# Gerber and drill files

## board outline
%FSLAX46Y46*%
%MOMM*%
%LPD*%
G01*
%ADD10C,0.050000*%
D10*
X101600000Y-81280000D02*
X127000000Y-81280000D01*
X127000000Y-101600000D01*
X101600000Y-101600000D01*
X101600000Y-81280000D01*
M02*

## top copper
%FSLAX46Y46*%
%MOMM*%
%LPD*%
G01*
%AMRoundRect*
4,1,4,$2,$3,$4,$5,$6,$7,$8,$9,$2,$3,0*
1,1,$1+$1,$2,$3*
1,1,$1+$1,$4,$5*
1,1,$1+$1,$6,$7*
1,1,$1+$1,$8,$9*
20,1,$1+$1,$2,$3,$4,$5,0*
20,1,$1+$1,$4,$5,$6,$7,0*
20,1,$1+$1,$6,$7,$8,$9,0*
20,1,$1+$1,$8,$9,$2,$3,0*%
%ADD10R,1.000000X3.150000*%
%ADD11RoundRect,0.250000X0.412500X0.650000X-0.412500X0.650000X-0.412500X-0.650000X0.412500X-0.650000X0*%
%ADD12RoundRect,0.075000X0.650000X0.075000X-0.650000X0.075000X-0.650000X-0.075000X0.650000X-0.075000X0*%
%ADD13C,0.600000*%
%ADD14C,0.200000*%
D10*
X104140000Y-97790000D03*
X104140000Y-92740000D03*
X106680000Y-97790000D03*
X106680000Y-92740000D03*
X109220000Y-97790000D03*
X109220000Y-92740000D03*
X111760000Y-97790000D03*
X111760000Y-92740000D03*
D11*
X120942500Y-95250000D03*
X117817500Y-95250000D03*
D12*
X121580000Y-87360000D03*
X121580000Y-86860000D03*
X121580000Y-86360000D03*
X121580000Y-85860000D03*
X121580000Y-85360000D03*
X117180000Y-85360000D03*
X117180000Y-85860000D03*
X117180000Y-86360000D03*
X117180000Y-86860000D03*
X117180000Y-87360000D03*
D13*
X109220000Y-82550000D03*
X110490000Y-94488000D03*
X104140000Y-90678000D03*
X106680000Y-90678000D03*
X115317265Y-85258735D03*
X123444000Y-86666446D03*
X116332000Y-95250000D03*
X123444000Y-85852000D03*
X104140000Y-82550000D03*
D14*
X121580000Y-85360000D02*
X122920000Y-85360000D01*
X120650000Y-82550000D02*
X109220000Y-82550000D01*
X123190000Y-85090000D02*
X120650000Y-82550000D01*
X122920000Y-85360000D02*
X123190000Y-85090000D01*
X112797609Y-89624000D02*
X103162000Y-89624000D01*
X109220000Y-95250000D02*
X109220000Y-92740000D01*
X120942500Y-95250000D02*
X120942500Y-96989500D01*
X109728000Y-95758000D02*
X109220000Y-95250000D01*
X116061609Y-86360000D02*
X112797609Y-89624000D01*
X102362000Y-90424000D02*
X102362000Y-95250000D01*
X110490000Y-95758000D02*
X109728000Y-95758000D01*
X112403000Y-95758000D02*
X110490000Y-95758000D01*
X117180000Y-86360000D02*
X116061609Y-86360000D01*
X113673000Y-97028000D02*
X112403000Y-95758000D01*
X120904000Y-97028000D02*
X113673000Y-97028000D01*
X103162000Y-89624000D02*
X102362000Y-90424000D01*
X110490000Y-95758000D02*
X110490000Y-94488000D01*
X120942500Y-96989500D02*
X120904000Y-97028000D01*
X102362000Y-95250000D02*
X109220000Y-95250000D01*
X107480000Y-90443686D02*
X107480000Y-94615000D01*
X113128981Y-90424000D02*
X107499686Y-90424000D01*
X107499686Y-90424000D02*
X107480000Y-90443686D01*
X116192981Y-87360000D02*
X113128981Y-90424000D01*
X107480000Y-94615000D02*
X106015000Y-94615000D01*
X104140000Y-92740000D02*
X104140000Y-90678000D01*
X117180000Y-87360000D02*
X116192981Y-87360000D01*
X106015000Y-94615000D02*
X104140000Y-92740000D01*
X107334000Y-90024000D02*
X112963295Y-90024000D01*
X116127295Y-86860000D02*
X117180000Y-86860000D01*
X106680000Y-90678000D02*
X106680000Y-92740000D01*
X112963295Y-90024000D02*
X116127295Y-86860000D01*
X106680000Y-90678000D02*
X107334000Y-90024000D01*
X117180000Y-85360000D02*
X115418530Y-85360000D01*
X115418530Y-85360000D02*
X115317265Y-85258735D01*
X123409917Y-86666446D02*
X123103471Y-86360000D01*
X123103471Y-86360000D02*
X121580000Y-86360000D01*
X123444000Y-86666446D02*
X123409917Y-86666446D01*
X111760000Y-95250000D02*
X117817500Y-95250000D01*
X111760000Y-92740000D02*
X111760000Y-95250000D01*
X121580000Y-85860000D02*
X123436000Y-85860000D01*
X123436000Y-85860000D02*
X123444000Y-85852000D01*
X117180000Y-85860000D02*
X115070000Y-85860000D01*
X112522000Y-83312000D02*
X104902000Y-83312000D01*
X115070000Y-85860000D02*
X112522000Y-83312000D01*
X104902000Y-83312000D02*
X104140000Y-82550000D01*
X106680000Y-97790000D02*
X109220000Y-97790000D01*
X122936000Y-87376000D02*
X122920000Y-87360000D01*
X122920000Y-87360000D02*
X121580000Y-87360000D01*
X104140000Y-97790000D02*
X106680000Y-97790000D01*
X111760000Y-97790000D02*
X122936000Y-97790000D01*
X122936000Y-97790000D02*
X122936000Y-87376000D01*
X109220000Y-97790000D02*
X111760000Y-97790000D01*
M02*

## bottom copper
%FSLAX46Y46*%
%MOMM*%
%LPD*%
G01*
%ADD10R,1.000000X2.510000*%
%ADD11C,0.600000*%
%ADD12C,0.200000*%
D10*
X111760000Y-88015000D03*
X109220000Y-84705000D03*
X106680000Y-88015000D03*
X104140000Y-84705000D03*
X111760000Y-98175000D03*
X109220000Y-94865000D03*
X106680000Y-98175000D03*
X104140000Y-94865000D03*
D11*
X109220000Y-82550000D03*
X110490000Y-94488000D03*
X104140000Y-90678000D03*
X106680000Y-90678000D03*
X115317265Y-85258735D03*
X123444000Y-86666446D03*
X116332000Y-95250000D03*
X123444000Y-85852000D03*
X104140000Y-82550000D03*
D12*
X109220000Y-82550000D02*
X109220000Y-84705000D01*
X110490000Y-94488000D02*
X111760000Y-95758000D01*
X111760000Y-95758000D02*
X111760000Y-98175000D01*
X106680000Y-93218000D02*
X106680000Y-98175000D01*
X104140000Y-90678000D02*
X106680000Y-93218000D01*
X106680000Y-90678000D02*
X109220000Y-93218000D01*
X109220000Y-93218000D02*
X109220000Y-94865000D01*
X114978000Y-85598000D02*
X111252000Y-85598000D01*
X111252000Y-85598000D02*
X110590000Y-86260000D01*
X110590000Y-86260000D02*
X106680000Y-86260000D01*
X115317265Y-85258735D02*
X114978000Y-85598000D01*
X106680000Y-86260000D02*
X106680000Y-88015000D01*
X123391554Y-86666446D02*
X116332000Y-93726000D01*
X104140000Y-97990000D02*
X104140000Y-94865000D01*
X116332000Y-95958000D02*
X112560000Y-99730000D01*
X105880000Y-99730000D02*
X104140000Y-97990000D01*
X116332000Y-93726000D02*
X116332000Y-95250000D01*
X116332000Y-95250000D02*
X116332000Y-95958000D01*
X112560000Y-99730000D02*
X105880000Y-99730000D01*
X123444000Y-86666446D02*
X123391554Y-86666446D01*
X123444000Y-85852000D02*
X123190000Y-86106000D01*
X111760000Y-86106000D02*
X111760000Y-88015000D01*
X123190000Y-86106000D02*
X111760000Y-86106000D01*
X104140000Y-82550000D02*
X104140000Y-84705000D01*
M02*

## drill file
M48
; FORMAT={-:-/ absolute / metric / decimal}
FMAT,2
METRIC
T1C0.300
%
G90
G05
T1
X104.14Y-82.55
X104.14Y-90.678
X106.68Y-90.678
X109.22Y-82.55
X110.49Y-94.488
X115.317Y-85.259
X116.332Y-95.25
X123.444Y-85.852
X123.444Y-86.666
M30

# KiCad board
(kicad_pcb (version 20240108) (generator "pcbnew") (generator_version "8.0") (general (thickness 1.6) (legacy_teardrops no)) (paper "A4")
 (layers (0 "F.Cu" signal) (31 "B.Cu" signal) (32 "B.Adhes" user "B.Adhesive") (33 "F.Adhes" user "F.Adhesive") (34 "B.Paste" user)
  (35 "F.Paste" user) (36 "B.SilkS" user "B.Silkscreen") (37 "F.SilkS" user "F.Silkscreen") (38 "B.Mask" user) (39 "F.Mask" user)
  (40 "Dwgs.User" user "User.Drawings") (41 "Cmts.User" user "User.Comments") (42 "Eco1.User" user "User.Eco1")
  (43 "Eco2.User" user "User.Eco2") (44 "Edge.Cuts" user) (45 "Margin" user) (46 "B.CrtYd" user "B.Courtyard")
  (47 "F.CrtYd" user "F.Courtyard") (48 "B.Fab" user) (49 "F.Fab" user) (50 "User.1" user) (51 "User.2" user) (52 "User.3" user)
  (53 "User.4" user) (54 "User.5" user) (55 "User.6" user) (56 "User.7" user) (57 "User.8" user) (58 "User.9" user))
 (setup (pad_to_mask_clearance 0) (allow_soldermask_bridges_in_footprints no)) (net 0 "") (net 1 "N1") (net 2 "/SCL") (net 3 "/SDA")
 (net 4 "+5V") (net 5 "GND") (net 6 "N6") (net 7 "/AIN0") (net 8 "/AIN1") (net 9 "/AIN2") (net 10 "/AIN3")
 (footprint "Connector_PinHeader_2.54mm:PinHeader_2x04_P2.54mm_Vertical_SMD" (layer "F.Cu") (at 107.95 95.265 90)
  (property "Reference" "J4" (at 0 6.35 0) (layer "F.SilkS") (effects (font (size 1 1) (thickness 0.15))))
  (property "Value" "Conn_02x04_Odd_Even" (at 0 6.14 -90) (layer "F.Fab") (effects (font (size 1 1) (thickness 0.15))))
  (pad "1" smd rect (at -2.525 -3.81 90) (size 3.15 1) (layers "F.Cu" "F.Paste" "F.Mask") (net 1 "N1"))
  (pad "2" smd rect (at 2.525 -3.81 90) (size 3.15 1) (layers "F.Cu" "F.Paste" "F.Mask") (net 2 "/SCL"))
  (pad "3" smd rect (at -2.525 -1.27 90) (size 3.15 1) (layers "F.Cu" "F.Paste" "F.Mask") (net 1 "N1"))
  (pad "4" smd rect (at 2.525 -1.27 90) (size 3.15 1) (layers "F.Cu" "F.Paste" "F.Mask") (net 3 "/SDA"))
  (pad "5" smd rect (at -2.525 1.27 90) (size 3.15 1) (layers "F.Cu" "F.Paste" "F.Mask") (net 1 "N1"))
  (pad "6" smd rect (at 2.525 1.27 90) (size 3.15 1) (layers "F.Cu" "F.Paste" "F.Mask") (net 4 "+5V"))
  (pad "7" smd rect (at -2.525 3.81 90) (size 3.15 1) (layers "F.Cu" "F.Paste" "F.Mask") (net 1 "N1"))
  (pad "8" smd rect (at 2.525 3.81 90) (size 3.15 1) (layers "F.Cu" "F.Paste" "F.Mask") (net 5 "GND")))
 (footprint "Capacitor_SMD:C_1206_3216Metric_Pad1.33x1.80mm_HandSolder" (layer "F.Cu") (at 119.38 95.25 180)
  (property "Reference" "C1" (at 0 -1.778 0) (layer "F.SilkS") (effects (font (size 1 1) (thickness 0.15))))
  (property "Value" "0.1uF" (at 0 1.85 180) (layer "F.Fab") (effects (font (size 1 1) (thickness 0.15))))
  (pad "1" smd roundrect (at -1.5625 0 180) (size 1.325 1.8) (layers "F.Cu" "F.Paste" "F.Mask") (roundrect_rratio 0.188679) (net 4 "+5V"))
  (pad "2" smd roundrect (at 1.5625 0 180) (size 1.325 1.8) (layers "F.Cu" "F.Paste" "F.Mask") (roundrect_rratio 0.188679) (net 5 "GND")))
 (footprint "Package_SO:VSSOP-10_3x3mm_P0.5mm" (layer "F.Cu") (at 119.38 86.36 180)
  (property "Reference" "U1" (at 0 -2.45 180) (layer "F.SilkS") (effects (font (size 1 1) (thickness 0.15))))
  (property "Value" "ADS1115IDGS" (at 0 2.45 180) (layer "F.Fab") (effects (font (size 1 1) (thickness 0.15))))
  (pad "1" smd roundrect (at -2.2 -1 180) (size 1.45 0.3) (layers "F.Cu" "F.Paste" "F.Mask") (roundrect_rratio 0.25) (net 1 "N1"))
  (pad "2" smd roundrect (at -2.2 -0.5 180) (size 1.45 0.3) (layers "F.Cu" "F.Paste" "F.Mask") (roundrect_rratio 0.25) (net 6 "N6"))
  (pad "3" smd roundrect (at -2.2 0 180) (size 1.45 0.3) (layers "F.Cu" "F.Paste" "F.Mask") (roundrect_rratio 0.25) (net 5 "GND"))
  (pad "4" smd roundrect (at -2.2 0.5 180) (size 1.45 0.3) (layers "F.Cu" "F.Paste" "F.Mask") (roundrect_rratio 0.25) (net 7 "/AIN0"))
  (pad "5" smd roundrect (at -2.2 1 180) (size 1.45 0.3) (layers "F.Cu" "F.Paste" "F.Mask") (roundrect_rratio 0.25) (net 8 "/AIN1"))
  (pad "6" smd roundrect (at 2.2 1 180) (size 1.45 0.3) (layers "F.Cu" "F.Paste" "F.Mask") (roundrect_rratio 0.25) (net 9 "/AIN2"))
  (pad "7" smd roundrect (at 2.2 0.5 180) (size 1.45 0.3) (layers "F.Cu" "F.Paste" "F.Mask") (roundrect_rratio 0.25) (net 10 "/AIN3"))
  (pad "8" smd roundrect (at 2.2 0 180) (size 1.45 0.3) (layers "F.Cu" "F.Paste" "F.Mask") (roundrect_rratio 0.25) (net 4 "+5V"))
  (pad "9" smd roundrect (at 2.2 -0.5 180) (size 1.45 0.3) (layers "F.Cu" "F.Paste" "F.Mask") (roundrect_rratio 0.25) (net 3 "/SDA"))
  (pad "10" smd roundrect (at 2.2 -1 180) (size 1.45 0.3) (layers "F.Cu" "F.Paste" "F.Mask") (roundrect_rratio 0.25) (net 2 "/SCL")))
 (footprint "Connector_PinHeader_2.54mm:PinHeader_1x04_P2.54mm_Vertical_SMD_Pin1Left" (layer "B.Cu") (at 107.95 86.36 90)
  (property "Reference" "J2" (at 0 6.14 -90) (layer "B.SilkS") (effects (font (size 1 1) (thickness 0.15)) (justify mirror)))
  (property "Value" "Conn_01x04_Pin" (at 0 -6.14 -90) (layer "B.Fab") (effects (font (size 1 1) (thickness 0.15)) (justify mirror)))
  (pad "1" smd rect (at -1.655 3.81 90) (size 2.51 1) (layers "B.Cu" "B.Paste" "B.Mask") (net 7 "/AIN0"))
  (pad "2" smd rect (at 1.655 1.27 90) (size 2.51 1) (layers "B.Cu" "B.Paste" "B.Mask") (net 8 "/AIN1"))
  (pad "3" smd rect (at -1.655 -1.27 90) (size 2.51 1) (layers "B.Cu" "B.Paste" "B.Mask") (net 9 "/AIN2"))
  (pad "4" smd rect (at 1.655 -3.81 90) (size 2.51 1) (layers "B.Cu" "B.Paste" "B.Mask") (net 10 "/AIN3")))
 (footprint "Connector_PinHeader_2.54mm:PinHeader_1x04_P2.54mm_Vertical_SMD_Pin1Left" (layer "B.Cu") (at 107.95 96.52 90)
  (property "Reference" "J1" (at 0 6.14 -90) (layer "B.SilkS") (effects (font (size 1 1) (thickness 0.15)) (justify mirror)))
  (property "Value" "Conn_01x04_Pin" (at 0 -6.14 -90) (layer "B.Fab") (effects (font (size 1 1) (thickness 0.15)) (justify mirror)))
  (pad "1" smd rect (at -1.655 3.81 90) (size 2.51 1) (layers "B.Cu" "B.Paste" "B.Mask") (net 4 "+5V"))
  (pad "2" smd rect (at 1.655 1.27 90) (size 2.51 1) (layers "B.Cu" "B.Paste" "B.Mask") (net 3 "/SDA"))
  (pad "3" smd rect (at -1.655 -1.27 90) (size 2.51 1) (layers "B.Cu" "B.Paste" "B.Mask") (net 2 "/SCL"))
  (pad "4" smd rect (at 1.655 -3.81 90) (size 2.51 1) (layers "B.Cu" "B.Paste" "B.Mask") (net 5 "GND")))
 (gr_rect (start 101.6 81.28) (end 127 101.6) (stroke (width 0.05) (type default)) (fill none) (layer "Edge.Cuts"))
 (segment (start 121.58 85.36) (end 122.92 85.36) (width 0.2) (layer "F.Cu") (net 8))
 (segment (start 120.65 82.55) (end 109.22 82.55) (width 0.2) (layer "F.Cu") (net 8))
 (segment (start 123.19 85.09) (end 120.65 82.55) (width 0.2) (layer "F.Cu") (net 8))
 (segment (start 122.92 85.36) (end 123.19 85.09) (width 0.2) (layer "F.Cu") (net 8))
 (via (at 109.22 82.55) (size 0.6) (drill 0.3) (layers "F.Cu" "B.Cu") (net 8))
 (segment (start 109.22 82.55) (end 109.22 84.705) (width 0.2) (layer "B.Cu") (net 8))
 (segment (start 112.797609 89.624) (end 103.162 89.624) (width 0.2) (layer "F.Cu") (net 4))
 (segment (start 109.22 95.25) (end 109.22 92.74) (width 0.2) (layer "F.Cu") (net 4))
 (segment (start 120.9425 95.25) (end 120.9425 96.9895) (width 0.2) (layer "F.Cu") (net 4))
 (segment (start 109.728 95.758) (end 109.22 95.25) (width 0.2) (layer "F.Cu") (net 4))
 (segment (start 116.061609 86.36) (end 112.797609 89.624) (width 0.2) (layer "F.Cu") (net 4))
 (segment (start 102.362 90.424) (end 102.362 95.25) (width 0.2) (layer "F.Cu") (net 4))
 (segment (start 110.49 95.758) (end 109.728 95.758) (width 0.2) (layer "F.Cu") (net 4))
 (segment (start 112.403 95.758) (end 110.49 95.758) (width 0.2) (layer "F.Cu") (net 4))
 (segment (start 117.18 86.36) (end 116.061609 86.36) (width 0.2) (layer "F.Cu") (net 4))
 (segment (start 113.673 97.028) (end 112.403 95.758) (width 0.2) (layer "F.Cu") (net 4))
 (segment (start 120.904 97.028) (end 113.673 97.028) (width 0.2) (layer "F.Cu") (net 4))
 (segment (start 103.162 89.624) (end 102.362 90.424) (width 0.2) (layer "F.Cu") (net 4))
 (segment (start 110.49 95.758) (end 110.49 94.488) (width 0.2) (layer "F.Cu") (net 4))
 (segment (start 120.9425 96.9895) (end 120.904 97.028) (width 0.2) (layer "F.Cu") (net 4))
 (segment (start 102.362 95.25) (end 109.22 95.25) (width 0.2) (layer "F.Cu") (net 4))
 (via (at 110.49 94.488) (size 0.6) (drill 0.3) (layers "F.Cu" "B.Cu") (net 4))
 (segment (start 110.49 94.488) (end 111.76 95.758) (width 0.2) (layer "B.Cu") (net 4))
 (segment (start 111.76 95.758) (end 111.76 98.175) (width 0.2) (layer "B.Cu") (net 4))
 (segment (start 107.48 90.443686) (end 107.48 94.615) (width 0.2) (layer "F.Cu") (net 2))
 (segment (start 113.128981 90.424) (end 107.499686 90.424) (width 0.2) (layer "F.Cu") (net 2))
 (segment (start 107.499686 90.424) (end 107.48 90.443686) (width 0.2) (layer "F.Cu") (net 2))
 (segment (start 116.192981 87.36) (end 113.128981 90.424) (width 0.2) (layer "F.Cu") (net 2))
 (segment (start 107.48 94.615) (end 106.015 94.615) (width 0.2) (layer "F.Cu") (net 2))
 (segment (start 104.14 92.74) (end 104.14 90.678) (width 0.2) (layer "F.Cu") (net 2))
 (segment (start 117.18 87.36) (end 116.192981 87.36) (width 0.2) (layer "F.Cu") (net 2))
 (segment (start 106.015 94.615) (end 104.14 92.74) (width 0.2) (layer "F.Cu") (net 2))
 (via (at 104.14 90.678) (size 0.6) (drill 0.3) (layers "F.Cu" "B.Cu") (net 2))
 (segment (start 106.68 93.218) (end 106.68 98.175) (width 0.2) (layer "B.Cu") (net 2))
 (segment (start 104.14 90.678) (end 106.68 93.218) (width 0.2) (layer "B.Cu") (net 2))
 (segment (start 107.334 90.024) (end 112.963295 90.024) (width 0.2) (layer "F.Cu") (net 3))
 (segment (start 116.127295 86.86) (end 117.18 86.86) (width 0.2) (layer "F.Cu") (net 3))
 (segment (start 106.68 90.678) (end 106.68 92.74) (width 0.2) (layer "F.Cu") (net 3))
 (segment (start 112.963295 90.024) (end 116.127295 86.86) (width 0.2) (layer "F.Cu") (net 3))
 (segment (start 106.68 90.678) (end 107.334 90.024) (width 0.2) (layer "F.Cu") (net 3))
 (via (at 106.68 90.678) (size 0.6) (drill 0.3) (layers "F.Cu" "B.Cu") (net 3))
 (segment (start 106.68 90.678) (end 109.22 93.218) (width 0.2) (layer "B.Cu") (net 3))
 (segment (start 109.22 93.218) (end 109.22 94.865) (width 0.2) (layer "B.Cu") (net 3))
 (segment (start 117.18 85.36) (end 115.41853 85.36) (width 0.2) (layer "F.Cu") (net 9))
 (segment (start 115.41853 85.36) (end 115.317265 85.258735) (width 0.2) (layer "F.Cu") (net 9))
 (via (at 115.317265 85.258735) (size 0.6) (drill 0.3) (layers "F.Cu" "B.Cu") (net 9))
 (segment (start 114.978 85.598) (end 111.252 85.598) (width 0.2) (layer "B.Cu") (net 9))
 (segment (start 111.252 85.598) (end 110.59 86.26) (width 0.2) (layer "B.Cu") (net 9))
 (segment (start 110.59 86.26) (end 106.68 86.26) (width 0.2) (layer "B.Cu") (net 9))
 (segment (start 115.317265 85.258735) (end 114.978 85.598) (width 0.2) (layer "B.Cu") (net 9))
 (segment (start 106.68 86.26) (end 106.68 88.015) (width 0.2) (layer "B.Cu") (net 9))
 (segment (start 123.409917 86.666446) (end 123.103471 86.36) (width 0.2) (layer "F.Cu") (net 5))
 (segment (start 123.103471 86.36) (end 121.58 86.36) (width 0.2) (layer "F.Cu") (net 5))
 (segment (start 123.444 86.666446) (end 123.409917 86.666446) (width 0.2) (layer "F.Cu") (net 5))
 (segment (start 111.76 95.25) (end 117.8175 95.25) (width 0.2) (layer "F.Cu") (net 5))
 (segment (start 111.76 92.74) (end 111.76 95.25) (width 0.2) (layer "F.Cu") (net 5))
 (via (at 123.444 86.666446) (size 0.6) (drill 0.3) (layers "F.Cu" "B.Cu") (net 5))
 (via (at 116.332 95.25) (size 0.6) (drill 0.3) (layers "F.Cu" "B.Cu") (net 5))
 (segment (start 123.391554 86.666446) (end 116.332 93.726) (width 0.2) (layer "B.Cu") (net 5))
 (segment (start 104.14 97.99) (end 104.14 94.865) (width 0.2) (layer "B.Cu") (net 5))
 (segment (start 116.332 95.958) (end 112.56 99.73) (width 0.2) (layer "B.Cu") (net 5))
 (segment (start 105.88 99.73) (end 104.14 97.99) (width 0.2) (layer "B.Cu") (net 5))
 (segment (start 116.332 93.726) (end 116.332 95.25) (width 0.2) (layer "B.Cu") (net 5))
 (segment (start 116.332 95.25) (end 116.332 95.958) (width 0.2) (layer "B.Cu") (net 5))
 (segment (start 112.56 99.73) (end 105.88 99.73) (width 0.2) (layer "B.Cu") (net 5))
 (segment (start 123.444 86.666446) (end 123.391554 86.666446) (width 0.2) (layer "B.Cu") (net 5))
 (segment (start 121.58 85.86) (end 123.436 85.86) (width 0.2) (layer "F.Cu") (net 7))
 (segment (start 123.436 85.86) (end 123.444 85.852) (width 0.2) (layer "F.Cu") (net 7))
 (via (at 123.444 85.852) (size 0.6) (drill 0.3) (layers "F.Cu" "B.Cu") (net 7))
 (segment (start 123.444 85.852) (end 123.19 86.106) (width 0.2) (layer "B.Cu") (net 7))
 (segment (start 111.76 86.106) (end 111.76 88.015) (width 0.2) (layer "B.Cu") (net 7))
 (segment (start 123.19 86.106) (end 111.76 86.106) (width 0.2) (layer "B.Cu") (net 7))
 (segment (start 117.18 85.86) (end 115.07 85.86) (width 0.2) (layer "F.Cu") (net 10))
 (segment (start 112.522 83.312) (end 104.902 83.312) (width 0.2) (layer "F.Cu") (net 10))
 (segment (start 115.07 85.86) (end 112.522 83.312) (width 0.2) (layer "F.Cu") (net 10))
 (segment (start 104.902 83.312) (end 104.14 82.55) (width 0.2) (layer "F.Cu") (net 10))
 (via (at 104.14 82.55) (size 0.6) (drill 0.3) (layers "F.Cu" "B.Cu") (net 10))
 (segment (start 104.14 82.55) (end 104.14 84.705) (width 0.2) (layer "B.Cu") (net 10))
 (segment (start 106.68 97.79) (end 109.22 97.79) (width 0.2) (layer "F.Cu") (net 1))
 (segment (start 122.936 87.376) (end 122.92 87.36) (width 0.2) (layer "F.Cu") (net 1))
 (segment (start 122.92 87.36) (end 121.58 87.36) (width 0.2) (layer "F.Cu") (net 1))
 (segment (start 104.14 97.79) (end 106.68 97.79) (width 0.2) (layer "F.Cu") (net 1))
 (segment (start 111.76 97.79) (end 122.936 97.79) (width 0.2) (layer "F.Cu") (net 1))
 (segment (start 122.936 97.79) (end 122.936 87.376) (width 0.2) (layer "F.Cu") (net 1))
 (segment (start 109.22 97.79) (end 111.76 97.79) (width 0.2) (layer "F.Cu") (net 1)))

